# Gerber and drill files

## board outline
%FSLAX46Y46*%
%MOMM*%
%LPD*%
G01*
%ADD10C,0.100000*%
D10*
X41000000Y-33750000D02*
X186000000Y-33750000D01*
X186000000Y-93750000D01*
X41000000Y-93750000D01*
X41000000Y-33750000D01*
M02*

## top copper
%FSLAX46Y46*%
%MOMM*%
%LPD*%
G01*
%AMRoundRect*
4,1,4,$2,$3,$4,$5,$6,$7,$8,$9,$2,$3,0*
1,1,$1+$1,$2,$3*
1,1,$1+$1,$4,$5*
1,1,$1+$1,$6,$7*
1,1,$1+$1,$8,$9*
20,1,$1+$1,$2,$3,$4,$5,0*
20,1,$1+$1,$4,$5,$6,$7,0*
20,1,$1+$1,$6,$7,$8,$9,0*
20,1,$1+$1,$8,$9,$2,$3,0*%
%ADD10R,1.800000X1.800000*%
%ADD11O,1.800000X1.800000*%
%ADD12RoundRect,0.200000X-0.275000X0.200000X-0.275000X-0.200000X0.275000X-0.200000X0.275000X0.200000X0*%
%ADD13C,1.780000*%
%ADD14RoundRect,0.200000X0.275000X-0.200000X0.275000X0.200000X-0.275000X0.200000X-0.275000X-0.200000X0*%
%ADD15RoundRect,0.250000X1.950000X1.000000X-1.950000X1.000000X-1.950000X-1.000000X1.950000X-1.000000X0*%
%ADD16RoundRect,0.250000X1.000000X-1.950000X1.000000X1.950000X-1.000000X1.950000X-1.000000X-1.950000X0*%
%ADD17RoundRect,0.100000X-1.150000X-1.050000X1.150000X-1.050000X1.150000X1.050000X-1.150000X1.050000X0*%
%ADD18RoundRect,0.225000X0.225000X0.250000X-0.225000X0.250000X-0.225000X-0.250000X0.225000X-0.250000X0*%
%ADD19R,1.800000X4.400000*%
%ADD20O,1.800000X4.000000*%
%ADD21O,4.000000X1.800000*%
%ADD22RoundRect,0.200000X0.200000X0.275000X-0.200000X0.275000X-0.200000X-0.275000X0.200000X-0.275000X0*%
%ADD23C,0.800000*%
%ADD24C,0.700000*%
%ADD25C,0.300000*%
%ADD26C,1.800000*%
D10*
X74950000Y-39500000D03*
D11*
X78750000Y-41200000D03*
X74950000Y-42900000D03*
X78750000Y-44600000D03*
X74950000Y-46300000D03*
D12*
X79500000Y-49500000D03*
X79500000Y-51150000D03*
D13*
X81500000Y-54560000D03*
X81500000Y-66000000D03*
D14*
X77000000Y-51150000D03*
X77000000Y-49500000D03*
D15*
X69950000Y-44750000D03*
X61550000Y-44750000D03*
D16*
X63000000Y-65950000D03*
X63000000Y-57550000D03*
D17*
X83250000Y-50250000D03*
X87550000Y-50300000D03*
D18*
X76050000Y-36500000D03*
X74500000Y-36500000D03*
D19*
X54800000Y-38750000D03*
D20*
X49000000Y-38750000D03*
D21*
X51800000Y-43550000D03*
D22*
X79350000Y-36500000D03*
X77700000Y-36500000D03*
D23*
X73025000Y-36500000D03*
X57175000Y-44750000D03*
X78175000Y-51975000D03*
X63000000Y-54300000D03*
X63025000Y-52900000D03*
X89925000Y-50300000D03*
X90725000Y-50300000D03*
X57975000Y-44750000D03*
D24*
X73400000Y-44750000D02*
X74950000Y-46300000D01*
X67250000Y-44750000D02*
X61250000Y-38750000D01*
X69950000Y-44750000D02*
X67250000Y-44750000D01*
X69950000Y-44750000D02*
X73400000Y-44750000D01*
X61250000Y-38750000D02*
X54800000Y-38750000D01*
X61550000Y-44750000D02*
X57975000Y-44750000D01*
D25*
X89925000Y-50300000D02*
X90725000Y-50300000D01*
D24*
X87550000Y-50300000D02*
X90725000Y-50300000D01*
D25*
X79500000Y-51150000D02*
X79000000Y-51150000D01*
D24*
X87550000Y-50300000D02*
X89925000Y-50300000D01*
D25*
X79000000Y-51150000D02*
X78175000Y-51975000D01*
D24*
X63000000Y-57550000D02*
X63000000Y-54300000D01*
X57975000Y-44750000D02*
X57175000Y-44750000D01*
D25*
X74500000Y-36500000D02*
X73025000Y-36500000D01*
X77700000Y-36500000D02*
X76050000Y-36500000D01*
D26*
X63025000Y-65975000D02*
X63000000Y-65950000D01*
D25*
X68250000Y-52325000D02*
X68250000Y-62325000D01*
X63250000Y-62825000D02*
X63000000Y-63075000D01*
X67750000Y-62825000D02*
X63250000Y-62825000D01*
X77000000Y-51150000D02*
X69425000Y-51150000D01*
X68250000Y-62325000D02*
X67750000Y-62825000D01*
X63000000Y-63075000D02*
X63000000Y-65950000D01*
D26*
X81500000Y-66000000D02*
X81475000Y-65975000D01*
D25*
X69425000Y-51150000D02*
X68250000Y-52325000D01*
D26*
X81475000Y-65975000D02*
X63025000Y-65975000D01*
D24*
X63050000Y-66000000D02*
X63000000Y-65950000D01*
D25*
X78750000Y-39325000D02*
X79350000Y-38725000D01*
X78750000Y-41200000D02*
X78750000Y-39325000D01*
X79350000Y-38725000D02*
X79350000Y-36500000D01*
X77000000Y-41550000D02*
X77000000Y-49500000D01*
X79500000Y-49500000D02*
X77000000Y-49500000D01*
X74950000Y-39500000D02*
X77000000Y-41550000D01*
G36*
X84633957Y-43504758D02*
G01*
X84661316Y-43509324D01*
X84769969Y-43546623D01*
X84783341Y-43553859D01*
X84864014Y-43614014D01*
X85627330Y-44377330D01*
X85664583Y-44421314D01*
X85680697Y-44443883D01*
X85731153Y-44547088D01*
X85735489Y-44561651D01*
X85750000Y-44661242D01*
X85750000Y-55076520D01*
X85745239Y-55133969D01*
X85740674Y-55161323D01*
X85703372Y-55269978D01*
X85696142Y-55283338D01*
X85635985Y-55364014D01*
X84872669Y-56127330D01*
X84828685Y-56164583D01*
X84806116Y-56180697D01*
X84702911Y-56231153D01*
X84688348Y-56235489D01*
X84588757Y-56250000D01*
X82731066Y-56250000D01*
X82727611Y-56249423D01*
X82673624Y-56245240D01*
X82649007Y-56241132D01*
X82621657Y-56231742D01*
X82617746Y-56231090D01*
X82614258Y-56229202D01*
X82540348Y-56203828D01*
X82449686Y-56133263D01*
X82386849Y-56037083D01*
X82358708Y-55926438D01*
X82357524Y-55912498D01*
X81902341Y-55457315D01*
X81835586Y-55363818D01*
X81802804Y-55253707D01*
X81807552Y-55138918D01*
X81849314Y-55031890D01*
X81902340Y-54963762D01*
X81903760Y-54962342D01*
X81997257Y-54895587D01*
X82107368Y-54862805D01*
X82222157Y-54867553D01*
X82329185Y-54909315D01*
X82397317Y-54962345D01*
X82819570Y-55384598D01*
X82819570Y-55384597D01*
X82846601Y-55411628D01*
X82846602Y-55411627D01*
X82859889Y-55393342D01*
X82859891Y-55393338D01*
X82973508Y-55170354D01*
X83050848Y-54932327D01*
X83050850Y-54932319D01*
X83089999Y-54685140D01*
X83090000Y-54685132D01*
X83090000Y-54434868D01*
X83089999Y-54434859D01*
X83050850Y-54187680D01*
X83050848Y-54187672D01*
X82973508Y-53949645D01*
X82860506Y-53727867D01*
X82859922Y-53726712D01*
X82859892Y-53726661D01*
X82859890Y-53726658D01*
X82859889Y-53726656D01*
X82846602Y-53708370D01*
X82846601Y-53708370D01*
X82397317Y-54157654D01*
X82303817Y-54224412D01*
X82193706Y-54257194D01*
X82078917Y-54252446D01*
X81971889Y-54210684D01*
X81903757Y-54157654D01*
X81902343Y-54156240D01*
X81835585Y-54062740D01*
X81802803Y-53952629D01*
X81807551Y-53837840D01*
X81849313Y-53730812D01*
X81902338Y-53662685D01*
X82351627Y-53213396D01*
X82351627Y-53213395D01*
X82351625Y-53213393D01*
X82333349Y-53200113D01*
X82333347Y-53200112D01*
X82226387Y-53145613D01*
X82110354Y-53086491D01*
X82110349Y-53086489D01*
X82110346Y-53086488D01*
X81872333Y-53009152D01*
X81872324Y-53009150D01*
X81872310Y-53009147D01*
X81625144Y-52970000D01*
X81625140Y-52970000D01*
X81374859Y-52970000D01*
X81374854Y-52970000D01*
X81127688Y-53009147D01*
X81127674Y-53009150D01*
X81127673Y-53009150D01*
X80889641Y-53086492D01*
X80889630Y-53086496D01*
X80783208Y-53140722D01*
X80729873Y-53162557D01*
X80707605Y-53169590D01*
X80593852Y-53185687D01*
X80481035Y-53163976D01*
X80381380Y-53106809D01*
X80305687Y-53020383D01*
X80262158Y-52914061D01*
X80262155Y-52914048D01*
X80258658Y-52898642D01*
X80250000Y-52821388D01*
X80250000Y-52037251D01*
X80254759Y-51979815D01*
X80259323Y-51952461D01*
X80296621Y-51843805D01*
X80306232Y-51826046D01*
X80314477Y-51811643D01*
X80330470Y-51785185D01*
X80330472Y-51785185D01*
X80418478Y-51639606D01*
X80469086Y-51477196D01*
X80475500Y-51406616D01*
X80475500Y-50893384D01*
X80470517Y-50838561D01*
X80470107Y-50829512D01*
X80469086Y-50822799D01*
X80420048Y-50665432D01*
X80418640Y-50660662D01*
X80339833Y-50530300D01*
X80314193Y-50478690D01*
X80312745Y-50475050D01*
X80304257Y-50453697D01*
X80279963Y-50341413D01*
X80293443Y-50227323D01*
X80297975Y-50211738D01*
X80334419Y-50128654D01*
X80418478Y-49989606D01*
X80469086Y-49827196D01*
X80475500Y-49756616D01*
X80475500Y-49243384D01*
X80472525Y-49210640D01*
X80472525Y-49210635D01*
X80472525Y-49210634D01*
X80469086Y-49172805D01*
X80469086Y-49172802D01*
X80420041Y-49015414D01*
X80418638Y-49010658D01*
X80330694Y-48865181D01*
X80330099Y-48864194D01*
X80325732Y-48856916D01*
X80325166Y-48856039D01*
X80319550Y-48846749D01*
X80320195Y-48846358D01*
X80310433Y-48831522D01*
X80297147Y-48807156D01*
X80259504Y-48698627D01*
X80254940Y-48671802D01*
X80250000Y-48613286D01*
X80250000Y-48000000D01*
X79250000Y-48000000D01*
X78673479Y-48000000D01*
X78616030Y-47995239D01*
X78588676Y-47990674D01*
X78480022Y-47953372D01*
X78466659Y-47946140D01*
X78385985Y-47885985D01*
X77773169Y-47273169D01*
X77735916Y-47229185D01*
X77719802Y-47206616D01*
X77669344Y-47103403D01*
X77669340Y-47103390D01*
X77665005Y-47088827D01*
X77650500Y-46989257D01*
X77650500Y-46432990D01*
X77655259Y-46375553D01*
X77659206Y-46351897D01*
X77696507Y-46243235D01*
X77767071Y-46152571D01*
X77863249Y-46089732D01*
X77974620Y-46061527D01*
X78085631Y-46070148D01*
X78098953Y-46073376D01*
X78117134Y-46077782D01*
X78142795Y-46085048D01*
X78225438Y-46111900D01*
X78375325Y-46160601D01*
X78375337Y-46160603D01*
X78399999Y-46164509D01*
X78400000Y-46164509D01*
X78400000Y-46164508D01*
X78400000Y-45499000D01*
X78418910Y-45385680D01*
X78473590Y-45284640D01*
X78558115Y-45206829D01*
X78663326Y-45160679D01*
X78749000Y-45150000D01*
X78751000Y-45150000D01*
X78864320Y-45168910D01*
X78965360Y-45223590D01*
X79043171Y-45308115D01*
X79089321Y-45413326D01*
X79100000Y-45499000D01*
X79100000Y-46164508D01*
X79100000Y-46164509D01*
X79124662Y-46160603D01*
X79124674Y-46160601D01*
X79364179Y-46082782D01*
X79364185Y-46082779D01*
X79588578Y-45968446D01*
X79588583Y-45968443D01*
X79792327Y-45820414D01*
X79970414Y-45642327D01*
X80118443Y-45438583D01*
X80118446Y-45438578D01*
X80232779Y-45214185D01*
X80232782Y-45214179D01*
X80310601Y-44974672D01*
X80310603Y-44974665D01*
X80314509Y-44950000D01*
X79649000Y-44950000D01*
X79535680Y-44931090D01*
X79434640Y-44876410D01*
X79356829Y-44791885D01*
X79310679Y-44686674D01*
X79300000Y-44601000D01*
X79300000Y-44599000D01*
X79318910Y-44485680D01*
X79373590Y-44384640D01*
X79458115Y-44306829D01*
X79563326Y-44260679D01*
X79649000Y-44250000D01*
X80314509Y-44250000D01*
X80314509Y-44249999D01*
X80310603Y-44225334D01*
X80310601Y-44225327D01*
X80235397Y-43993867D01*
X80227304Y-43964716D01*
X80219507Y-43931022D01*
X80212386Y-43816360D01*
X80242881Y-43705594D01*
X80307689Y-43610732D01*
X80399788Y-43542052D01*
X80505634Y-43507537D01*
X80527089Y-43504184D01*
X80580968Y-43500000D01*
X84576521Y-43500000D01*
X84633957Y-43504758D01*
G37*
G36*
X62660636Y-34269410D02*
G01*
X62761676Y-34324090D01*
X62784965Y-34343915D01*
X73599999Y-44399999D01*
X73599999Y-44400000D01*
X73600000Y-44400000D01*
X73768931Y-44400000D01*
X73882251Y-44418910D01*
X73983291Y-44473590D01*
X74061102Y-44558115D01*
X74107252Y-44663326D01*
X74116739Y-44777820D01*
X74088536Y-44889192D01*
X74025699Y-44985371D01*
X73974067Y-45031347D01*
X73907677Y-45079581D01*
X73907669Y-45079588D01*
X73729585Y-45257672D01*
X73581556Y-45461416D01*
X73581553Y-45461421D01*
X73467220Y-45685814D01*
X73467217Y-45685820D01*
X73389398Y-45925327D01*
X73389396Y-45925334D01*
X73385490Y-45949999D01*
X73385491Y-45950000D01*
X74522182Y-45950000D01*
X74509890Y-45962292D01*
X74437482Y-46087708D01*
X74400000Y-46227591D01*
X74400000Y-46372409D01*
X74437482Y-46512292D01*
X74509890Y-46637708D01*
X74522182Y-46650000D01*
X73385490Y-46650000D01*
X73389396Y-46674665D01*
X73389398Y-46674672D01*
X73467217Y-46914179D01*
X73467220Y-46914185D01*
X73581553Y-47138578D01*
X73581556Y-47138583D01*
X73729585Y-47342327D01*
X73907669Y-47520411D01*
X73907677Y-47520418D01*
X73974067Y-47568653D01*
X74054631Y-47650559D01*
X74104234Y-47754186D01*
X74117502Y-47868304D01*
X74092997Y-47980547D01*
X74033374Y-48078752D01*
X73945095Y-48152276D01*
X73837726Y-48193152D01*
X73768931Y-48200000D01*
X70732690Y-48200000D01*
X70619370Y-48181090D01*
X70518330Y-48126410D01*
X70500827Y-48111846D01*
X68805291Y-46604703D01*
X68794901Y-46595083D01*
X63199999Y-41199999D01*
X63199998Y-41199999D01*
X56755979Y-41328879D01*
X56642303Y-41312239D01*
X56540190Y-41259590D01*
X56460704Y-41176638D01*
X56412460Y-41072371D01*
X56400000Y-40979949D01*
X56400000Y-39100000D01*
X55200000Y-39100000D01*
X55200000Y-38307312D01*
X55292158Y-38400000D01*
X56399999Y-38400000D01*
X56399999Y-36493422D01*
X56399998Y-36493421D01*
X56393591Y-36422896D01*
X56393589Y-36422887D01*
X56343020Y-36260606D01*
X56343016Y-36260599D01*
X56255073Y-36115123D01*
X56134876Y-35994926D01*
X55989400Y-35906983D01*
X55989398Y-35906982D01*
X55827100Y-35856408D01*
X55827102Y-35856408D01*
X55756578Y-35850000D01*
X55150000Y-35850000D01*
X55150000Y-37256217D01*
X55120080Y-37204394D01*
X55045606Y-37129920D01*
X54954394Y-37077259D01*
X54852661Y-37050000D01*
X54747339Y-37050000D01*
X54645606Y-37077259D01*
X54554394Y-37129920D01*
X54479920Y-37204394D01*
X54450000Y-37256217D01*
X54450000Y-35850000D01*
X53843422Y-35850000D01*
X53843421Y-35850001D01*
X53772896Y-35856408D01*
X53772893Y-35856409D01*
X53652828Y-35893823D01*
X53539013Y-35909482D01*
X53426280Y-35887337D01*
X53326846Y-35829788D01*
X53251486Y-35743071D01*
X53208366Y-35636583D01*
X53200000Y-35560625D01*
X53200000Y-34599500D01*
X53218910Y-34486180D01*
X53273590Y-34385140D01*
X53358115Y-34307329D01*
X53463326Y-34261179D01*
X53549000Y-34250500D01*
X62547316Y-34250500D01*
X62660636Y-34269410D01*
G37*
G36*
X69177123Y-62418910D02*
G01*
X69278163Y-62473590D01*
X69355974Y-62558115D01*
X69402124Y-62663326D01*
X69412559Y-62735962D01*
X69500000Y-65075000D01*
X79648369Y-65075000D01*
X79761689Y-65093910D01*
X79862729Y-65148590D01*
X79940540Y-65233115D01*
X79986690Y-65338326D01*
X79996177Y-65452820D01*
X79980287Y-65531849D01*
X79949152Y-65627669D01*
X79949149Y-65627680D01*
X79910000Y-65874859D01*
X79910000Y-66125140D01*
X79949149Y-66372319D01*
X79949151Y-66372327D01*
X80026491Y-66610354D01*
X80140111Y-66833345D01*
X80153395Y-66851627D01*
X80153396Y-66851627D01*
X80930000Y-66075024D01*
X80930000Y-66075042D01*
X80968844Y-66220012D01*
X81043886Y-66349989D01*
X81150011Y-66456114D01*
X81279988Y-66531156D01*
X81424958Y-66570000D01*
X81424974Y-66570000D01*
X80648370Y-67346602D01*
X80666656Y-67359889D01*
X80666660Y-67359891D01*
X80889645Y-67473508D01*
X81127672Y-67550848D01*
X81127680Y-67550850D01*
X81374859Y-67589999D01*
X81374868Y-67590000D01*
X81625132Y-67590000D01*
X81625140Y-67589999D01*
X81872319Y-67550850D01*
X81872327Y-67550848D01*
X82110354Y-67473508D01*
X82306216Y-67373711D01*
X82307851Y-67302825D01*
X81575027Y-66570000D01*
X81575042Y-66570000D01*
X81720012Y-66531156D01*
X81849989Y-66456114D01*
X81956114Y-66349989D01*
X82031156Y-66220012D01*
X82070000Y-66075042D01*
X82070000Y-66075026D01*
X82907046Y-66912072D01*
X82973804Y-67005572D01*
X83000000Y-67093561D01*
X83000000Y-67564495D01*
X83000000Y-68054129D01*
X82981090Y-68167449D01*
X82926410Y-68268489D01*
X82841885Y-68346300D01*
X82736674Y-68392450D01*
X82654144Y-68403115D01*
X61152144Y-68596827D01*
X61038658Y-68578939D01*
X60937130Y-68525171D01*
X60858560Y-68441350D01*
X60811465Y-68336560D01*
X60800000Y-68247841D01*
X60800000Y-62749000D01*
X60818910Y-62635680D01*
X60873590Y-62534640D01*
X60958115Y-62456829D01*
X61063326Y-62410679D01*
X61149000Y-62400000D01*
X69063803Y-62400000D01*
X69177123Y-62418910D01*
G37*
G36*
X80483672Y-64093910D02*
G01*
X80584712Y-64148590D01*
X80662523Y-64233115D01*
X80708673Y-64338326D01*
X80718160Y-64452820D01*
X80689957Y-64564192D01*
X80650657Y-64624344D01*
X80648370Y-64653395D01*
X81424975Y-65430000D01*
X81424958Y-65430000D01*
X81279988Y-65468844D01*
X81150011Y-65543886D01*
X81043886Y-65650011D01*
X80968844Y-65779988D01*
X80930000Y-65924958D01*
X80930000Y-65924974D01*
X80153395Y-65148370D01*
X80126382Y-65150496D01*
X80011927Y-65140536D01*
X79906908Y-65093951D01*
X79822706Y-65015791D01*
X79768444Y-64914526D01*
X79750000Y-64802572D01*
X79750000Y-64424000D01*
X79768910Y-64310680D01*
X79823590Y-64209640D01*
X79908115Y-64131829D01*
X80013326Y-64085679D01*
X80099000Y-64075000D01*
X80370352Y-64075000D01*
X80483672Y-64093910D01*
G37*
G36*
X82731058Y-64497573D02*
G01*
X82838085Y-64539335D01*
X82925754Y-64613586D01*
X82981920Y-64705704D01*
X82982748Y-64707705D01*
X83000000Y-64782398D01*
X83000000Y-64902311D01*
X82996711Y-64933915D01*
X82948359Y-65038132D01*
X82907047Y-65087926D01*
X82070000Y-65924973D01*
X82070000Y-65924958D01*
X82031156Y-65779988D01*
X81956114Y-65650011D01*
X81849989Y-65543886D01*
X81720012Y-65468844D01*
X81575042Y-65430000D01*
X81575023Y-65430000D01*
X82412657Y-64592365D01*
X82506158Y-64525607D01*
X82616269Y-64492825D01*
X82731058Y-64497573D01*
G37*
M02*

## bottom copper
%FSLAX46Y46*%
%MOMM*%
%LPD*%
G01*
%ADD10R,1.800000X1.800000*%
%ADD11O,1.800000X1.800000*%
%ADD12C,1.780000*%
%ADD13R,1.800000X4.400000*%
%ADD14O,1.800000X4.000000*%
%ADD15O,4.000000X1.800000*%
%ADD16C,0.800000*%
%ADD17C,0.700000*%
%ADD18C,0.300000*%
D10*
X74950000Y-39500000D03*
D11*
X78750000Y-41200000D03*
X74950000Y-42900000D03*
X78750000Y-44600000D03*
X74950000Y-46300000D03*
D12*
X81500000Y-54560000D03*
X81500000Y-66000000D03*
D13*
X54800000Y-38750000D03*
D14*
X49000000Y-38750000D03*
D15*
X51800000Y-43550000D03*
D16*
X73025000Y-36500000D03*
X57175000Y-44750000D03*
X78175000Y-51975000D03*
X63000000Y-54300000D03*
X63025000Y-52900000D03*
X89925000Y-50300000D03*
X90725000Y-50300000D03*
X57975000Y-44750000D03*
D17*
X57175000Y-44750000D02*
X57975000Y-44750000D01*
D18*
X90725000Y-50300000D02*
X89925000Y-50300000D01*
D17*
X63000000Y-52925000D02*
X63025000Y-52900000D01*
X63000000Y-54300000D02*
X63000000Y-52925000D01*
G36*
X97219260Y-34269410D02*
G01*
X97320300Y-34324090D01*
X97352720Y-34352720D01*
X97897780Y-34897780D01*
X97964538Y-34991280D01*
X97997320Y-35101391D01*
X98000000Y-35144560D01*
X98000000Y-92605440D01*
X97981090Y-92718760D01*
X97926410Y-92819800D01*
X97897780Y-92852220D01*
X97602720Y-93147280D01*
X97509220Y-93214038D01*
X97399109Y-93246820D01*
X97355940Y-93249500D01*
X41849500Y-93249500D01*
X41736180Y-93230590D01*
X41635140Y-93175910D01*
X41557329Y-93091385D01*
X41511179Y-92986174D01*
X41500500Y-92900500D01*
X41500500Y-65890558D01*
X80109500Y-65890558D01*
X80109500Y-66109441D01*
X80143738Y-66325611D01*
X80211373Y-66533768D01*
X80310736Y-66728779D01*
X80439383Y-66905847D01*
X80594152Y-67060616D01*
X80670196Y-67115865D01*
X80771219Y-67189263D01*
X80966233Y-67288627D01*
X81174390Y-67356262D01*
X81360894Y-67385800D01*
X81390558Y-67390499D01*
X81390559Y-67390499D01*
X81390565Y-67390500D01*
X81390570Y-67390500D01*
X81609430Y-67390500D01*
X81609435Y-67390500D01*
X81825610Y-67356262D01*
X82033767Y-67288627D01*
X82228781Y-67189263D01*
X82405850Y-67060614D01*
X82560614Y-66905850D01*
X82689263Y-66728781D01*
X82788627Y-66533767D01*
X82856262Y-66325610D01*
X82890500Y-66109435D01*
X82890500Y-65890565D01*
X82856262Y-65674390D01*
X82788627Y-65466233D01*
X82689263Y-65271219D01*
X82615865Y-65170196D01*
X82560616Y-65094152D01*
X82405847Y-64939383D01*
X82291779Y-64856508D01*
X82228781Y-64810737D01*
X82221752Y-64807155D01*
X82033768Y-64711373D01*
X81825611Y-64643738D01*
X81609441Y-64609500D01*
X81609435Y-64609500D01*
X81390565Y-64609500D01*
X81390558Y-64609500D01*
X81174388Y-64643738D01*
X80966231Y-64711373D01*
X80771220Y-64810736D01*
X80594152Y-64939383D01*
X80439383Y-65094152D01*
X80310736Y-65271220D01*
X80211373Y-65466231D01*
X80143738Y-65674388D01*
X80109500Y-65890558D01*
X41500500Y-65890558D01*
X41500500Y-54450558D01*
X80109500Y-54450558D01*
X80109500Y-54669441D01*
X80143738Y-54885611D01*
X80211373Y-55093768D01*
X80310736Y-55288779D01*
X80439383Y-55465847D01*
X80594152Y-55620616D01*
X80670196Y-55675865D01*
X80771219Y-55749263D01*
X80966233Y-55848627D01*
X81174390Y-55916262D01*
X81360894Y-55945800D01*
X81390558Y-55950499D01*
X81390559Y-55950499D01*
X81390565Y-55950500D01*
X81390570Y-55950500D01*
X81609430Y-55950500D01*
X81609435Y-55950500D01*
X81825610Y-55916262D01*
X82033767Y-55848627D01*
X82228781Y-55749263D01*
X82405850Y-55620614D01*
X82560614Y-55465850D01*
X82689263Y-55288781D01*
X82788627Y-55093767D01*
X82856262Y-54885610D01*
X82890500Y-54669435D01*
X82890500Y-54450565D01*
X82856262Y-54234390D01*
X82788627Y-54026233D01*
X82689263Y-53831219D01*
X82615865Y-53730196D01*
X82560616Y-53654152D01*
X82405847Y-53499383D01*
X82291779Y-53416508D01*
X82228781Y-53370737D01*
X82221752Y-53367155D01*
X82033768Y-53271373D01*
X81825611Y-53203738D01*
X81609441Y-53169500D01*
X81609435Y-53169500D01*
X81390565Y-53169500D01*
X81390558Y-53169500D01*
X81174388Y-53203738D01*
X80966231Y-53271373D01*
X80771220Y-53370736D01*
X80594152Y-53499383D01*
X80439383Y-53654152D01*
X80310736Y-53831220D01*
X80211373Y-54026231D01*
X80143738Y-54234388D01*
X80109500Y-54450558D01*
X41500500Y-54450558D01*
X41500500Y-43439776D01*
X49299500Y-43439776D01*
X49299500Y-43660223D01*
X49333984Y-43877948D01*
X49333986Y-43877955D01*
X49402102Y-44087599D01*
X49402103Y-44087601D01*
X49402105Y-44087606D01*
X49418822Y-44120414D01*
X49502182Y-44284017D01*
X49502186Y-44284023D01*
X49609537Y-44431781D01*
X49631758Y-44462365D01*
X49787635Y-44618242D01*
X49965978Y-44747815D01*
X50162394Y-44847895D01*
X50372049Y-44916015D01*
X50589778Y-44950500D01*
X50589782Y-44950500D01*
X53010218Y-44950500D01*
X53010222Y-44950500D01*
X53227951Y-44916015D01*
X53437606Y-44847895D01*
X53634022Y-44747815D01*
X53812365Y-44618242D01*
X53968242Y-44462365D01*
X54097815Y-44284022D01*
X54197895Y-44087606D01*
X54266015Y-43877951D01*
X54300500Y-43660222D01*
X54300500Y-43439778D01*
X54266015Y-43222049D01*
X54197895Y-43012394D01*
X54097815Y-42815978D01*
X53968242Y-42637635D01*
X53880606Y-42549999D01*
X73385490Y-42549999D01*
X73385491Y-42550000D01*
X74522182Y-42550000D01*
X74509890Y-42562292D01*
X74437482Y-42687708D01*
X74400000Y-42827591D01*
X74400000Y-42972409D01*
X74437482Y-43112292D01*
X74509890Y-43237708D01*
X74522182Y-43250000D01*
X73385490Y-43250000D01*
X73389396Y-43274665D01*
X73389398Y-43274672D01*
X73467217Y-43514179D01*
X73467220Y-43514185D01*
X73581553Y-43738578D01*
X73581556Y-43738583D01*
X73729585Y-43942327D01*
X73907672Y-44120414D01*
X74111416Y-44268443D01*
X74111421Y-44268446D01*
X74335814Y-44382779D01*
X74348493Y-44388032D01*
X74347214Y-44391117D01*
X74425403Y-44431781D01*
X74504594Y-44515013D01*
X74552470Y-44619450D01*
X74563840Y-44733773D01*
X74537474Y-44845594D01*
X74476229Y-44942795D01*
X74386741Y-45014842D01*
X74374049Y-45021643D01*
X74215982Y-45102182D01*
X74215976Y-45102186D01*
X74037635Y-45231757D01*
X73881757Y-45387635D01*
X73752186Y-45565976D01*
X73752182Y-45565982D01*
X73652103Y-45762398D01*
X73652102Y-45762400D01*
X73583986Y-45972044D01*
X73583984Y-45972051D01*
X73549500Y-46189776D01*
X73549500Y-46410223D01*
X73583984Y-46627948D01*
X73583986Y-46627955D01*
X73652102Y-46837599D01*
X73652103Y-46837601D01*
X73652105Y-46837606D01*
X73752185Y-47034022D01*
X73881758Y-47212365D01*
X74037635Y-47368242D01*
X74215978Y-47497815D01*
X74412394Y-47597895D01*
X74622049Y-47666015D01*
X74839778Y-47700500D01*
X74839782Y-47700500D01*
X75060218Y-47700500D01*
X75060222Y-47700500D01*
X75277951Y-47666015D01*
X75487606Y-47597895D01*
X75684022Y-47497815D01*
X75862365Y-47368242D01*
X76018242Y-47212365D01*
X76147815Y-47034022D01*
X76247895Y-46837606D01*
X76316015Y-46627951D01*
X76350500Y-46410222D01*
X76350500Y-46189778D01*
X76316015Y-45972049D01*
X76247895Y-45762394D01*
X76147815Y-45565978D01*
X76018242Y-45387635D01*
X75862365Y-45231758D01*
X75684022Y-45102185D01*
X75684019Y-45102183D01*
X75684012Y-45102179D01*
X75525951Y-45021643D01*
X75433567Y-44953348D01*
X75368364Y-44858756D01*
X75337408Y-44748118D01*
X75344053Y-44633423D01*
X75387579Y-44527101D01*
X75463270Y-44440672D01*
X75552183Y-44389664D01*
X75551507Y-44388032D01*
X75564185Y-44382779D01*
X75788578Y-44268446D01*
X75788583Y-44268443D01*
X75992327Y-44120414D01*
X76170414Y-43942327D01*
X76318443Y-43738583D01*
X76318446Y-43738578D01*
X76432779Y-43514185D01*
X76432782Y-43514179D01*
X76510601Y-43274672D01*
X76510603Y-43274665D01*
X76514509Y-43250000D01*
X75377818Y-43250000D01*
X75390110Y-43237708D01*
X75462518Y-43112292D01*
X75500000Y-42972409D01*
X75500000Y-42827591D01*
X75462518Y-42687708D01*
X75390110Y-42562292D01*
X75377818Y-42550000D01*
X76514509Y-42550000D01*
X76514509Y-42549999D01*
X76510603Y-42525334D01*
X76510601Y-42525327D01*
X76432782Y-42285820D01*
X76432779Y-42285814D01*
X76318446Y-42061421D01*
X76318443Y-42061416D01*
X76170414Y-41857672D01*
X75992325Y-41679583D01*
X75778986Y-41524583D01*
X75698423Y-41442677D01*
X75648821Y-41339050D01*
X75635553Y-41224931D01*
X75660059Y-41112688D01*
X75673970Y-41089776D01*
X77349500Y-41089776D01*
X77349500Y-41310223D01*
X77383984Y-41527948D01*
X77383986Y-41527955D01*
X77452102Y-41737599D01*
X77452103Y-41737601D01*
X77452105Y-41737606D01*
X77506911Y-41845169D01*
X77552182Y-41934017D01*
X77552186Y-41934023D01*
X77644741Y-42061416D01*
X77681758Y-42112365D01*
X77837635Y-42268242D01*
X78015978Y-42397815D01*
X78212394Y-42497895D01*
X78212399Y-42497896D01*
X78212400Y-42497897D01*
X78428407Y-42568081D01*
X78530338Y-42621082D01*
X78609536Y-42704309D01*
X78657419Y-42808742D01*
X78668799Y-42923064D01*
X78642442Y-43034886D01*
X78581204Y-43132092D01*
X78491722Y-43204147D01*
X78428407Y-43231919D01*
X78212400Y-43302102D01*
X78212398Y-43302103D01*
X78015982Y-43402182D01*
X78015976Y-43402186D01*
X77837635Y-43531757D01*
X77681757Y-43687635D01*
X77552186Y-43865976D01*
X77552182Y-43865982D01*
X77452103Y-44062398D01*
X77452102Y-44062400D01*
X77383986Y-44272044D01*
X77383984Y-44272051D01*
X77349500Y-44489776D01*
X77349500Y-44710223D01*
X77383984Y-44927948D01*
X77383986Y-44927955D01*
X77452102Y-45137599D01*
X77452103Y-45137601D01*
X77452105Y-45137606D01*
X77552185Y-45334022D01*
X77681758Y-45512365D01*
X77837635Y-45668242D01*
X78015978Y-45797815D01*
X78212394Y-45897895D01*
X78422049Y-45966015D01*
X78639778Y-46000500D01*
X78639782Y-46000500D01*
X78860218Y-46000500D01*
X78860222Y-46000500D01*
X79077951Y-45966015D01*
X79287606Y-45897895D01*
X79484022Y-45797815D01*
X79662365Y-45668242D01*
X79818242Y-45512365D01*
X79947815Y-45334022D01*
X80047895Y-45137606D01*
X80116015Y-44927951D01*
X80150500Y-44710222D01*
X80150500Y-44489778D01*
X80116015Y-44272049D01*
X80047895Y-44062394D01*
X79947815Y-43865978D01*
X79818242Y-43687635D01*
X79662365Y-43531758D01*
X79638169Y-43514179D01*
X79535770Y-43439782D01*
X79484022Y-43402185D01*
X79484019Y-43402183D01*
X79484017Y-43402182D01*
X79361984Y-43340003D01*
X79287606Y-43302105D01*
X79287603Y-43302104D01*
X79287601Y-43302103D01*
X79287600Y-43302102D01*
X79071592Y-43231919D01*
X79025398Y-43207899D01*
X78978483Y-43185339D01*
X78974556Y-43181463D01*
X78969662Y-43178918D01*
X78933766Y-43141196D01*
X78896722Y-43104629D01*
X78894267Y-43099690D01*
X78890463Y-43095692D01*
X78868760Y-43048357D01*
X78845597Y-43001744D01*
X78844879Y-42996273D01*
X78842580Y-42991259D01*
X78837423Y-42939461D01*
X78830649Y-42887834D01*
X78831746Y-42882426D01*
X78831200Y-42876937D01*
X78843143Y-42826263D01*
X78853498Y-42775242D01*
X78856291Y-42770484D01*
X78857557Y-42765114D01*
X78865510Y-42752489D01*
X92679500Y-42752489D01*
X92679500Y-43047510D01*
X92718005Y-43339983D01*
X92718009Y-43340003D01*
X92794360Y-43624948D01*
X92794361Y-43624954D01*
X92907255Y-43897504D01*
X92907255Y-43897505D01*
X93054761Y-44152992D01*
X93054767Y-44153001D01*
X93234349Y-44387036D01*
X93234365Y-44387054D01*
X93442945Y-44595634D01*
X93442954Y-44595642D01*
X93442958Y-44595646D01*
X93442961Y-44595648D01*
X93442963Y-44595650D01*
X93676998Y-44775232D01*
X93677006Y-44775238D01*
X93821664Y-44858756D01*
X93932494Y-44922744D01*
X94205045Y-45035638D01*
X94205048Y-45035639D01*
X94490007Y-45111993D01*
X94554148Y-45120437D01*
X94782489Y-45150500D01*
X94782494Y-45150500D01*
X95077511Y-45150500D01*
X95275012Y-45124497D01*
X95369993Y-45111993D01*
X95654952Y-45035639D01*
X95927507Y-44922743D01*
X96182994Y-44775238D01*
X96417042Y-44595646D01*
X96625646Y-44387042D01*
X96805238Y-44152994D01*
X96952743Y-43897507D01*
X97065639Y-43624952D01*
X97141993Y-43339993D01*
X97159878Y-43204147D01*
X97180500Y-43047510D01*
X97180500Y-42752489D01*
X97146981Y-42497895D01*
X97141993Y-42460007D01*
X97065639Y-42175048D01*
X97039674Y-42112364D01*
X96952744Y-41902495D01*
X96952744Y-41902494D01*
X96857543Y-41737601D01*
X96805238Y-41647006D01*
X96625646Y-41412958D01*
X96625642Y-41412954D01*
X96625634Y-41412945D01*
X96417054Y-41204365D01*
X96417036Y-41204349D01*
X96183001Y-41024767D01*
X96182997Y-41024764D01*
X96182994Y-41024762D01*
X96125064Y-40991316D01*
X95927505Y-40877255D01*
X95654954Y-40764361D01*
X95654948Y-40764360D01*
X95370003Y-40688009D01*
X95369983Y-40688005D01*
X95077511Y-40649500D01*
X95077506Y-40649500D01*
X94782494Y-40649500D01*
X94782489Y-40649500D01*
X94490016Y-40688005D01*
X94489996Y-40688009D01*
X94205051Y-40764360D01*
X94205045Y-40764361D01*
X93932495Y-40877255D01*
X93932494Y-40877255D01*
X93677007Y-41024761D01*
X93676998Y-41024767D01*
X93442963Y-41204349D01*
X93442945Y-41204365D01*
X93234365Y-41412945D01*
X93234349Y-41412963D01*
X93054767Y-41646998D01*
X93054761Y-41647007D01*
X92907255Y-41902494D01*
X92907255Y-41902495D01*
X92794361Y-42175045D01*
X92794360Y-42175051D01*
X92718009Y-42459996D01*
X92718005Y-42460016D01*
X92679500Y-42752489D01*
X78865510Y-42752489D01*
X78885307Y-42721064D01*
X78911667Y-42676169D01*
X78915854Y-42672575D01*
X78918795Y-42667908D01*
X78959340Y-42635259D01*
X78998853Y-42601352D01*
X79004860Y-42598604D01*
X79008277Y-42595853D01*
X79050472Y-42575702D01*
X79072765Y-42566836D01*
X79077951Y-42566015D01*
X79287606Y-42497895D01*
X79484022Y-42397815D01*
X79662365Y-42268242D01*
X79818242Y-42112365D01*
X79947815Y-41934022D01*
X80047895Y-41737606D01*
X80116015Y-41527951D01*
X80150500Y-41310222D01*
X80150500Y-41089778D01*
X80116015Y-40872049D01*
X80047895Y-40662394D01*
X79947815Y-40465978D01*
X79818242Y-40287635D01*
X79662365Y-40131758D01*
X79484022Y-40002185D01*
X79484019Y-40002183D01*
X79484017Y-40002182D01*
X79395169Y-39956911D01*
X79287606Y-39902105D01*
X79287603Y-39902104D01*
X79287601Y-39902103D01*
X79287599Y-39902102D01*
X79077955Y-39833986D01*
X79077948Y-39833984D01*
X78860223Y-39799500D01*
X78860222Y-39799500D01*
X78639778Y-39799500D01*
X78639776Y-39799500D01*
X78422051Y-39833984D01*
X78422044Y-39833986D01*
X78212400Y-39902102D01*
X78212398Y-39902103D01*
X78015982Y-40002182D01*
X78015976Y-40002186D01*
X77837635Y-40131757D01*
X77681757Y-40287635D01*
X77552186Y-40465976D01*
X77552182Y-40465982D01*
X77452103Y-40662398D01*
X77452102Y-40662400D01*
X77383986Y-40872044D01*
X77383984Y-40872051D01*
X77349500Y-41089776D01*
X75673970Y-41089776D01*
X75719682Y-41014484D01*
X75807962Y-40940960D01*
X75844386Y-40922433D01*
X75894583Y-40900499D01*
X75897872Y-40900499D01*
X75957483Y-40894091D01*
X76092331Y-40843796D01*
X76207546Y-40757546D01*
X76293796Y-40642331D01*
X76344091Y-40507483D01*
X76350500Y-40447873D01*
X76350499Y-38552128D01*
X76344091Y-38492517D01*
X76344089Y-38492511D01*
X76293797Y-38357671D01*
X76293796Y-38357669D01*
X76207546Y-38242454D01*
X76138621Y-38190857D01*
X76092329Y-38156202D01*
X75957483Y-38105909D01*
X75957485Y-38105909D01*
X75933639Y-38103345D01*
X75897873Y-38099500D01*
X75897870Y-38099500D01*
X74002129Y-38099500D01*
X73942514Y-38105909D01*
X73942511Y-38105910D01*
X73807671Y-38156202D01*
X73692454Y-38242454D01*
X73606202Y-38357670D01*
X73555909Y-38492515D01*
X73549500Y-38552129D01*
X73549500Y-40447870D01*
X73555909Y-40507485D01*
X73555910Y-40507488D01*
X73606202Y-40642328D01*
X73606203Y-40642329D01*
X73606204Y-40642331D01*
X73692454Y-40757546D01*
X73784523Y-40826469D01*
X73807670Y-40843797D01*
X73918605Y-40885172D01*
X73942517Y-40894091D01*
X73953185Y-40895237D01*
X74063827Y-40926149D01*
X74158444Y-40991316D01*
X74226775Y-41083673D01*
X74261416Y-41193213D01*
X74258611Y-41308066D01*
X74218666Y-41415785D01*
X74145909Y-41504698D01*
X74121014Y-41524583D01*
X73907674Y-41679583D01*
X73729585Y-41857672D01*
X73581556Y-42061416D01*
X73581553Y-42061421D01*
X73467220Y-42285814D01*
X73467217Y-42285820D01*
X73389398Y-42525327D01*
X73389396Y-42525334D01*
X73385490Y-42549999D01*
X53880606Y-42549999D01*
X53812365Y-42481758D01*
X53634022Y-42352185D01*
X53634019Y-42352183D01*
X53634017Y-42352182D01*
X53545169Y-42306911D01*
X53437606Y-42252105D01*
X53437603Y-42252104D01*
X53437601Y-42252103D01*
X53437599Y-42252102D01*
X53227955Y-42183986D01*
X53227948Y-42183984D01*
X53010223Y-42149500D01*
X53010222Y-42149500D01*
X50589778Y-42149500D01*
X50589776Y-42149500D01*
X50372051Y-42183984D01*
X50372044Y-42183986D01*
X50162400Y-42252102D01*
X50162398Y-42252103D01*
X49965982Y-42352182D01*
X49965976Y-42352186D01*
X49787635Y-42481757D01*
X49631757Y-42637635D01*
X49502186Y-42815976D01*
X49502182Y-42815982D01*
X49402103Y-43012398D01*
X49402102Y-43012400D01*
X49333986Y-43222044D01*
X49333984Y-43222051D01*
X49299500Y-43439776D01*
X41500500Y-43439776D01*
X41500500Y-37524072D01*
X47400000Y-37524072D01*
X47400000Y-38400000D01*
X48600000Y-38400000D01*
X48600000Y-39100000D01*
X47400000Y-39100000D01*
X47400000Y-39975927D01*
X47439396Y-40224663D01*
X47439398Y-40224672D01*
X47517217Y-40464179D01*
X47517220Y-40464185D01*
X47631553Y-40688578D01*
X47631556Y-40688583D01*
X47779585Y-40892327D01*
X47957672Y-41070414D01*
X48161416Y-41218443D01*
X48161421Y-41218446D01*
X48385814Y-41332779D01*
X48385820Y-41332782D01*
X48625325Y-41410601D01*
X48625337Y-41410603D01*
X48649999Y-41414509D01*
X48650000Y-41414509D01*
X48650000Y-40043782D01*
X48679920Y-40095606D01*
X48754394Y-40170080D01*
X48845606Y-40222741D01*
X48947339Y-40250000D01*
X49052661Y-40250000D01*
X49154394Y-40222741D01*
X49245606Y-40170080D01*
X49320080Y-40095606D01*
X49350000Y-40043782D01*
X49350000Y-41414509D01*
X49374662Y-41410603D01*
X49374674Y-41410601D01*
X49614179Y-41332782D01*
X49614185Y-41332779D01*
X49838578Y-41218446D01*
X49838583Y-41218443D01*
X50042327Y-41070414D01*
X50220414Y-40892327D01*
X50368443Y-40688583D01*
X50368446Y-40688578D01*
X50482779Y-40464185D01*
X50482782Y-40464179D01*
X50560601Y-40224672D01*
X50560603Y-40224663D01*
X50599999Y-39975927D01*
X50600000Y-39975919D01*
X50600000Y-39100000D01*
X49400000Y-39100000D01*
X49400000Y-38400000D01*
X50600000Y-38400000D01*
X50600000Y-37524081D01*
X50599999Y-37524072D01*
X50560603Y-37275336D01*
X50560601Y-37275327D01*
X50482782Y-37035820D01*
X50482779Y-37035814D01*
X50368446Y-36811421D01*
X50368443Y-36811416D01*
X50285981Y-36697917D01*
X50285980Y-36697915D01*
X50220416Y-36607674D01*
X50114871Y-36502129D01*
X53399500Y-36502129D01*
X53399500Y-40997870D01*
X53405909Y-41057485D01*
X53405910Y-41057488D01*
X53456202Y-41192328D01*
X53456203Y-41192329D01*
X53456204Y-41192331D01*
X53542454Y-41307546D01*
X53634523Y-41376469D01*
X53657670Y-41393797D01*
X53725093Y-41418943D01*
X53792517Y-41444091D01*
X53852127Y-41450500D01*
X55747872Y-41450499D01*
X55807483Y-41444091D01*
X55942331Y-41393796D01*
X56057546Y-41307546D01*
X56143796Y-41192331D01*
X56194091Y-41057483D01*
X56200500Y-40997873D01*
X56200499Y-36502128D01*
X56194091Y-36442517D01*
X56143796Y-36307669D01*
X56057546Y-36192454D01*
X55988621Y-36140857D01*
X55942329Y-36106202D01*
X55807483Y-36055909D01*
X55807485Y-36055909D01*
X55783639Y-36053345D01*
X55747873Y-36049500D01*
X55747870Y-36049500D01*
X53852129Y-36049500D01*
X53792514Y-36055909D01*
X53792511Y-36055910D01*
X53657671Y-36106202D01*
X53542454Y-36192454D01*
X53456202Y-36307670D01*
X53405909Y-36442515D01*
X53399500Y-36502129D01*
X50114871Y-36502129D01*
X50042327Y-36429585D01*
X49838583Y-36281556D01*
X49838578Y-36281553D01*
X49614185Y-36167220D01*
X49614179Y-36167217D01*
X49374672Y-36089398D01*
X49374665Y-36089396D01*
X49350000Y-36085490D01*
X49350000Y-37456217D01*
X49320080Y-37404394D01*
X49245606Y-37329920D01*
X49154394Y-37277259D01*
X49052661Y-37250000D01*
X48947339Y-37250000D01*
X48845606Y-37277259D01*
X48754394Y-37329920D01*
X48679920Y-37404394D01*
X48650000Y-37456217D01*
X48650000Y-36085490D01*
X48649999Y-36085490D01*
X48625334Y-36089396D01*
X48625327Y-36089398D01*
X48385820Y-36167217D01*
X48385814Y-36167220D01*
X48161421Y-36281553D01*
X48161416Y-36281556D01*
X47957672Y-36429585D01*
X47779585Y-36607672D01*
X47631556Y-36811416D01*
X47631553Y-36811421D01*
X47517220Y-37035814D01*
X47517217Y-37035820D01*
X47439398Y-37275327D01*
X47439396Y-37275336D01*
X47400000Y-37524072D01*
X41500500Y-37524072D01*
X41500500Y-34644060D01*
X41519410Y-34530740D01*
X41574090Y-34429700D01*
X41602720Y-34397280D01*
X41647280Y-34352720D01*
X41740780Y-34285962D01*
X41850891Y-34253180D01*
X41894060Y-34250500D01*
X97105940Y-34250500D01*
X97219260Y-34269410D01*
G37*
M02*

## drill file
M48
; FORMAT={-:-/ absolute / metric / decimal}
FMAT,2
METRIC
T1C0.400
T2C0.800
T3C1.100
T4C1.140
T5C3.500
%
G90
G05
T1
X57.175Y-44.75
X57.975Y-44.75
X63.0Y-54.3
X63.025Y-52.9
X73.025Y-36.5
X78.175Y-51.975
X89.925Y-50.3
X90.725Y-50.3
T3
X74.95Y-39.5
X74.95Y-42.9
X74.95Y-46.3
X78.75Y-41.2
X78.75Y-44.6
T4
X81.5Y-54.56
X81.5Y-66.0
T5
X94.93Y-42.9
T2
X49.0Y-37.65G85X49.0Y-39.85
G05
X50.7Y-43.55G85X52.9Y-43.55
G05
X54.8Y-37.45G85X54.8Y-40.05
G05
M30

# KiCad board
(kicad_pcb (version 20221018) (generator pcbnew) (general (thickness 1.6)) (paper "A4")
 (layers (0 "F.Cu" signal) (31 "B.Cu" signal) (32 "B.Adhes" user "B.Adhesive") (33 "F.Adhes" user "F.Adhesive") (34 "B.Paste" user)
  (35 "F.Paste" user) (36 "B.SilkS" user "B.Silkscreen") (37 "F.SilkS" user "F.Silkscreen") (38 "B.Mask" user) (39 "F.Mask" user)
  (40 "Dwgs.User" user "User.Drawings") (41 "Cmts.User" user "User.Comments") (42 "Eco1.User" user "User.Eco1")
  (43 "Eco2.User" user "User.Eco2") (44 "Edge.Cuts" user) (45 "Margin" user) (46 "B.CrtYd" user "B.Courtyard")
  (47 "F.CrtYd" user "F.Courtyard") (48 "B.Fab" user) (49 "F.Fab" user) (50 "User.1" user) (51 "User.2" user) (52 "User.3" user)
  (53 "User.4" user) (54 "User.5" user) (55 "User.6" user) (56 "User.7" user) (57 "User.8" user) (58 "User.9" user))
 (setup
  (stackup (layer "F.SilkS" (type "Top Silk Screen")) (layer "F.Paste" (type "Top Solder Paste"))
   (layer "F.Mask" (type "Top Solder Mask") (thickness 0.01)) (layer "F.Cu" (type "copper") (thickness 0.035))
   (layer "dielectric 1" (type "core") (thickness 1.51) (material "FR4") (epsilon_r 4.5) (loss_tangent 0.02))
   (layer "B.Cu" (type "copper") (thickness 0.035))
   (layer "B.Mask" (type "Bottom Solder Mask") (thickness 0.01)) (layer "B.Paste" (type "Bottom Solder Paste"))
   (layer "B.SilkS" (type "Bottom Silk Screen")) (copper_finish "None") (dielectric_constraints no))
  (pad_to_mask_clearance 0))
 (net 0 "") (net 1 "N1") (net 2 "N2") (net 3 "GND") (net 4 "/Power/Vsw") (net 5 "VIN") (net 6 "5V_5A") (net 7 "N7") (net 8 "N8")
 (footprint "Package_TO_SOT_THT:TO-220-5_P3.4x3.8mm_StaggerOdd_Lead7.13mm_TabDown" (layer "F.Cu") (at 74.95 39.5 -90)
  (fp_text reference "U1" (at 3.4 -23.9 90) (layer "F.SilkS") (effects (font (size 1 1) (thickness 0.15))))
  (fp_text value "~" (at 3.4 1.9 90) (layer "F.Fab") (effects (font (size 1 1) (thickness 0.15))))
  (pad "" np_thru_hole oval (at 3.4 -19.98 270) (size 3.5 3.5) (drill 3.5) (layers "*.Cu" "*.Mask"))
  (pad "1" thru_hole rect (at 0 0 270) (size 1.8 1.8) (drill 1.1) (layers "*.Cu" "*.Mask") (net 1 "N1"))
  (pad "2" thru_hole oval (at 1.7 -3.8 270) (size 1.8 1.8) (drill 1.1) (layers "*.Cu" "*.Mask") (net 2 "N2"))
  (pad "3" thru_hole oval (at 3.4 0 270) (size 1.8 1.8) (drill 1.1) (layers "*.Cu" "*.Mask") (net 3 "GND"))
  (pad "4" thru_hole oval (at 5.1 -3.8 270) (size 1.8 1.8) (drill 1.1) (layers "*.Cu" "*.Mask") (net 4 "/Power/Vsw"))
  (pad "5" thru_hole oval (at 6.8 0 270) (size 1.8 1.8) (drill 1.1) (layers "*.Cu" "*.Mask") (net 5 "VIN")))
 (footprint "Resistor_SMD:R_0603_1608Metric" (layer "F.Cu") (at 79.5 50.325 -90)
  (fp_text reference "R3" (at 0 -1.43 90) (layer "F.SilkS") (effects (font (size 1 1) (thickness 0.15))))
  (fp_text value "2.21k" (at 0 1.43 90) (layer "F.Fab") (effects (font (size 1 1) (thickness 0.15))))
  (pad "1" smd roundrect (at -0.825 0 270) (size 0.8 0.95) (layers "F.Cu" "F.Paste" "F.Mask") (roundrect_rratio 0.25) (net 1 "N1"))
  (pad "2" smd roundrect (at 0.825 0 270) (size 0.8 0.95) (layers "F.Cu" "F.Paste" "F.Mask") (roundrect_rratio 0.25) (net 3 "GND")))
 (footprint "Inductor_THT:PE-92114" (layer "F.Cu") (at 81.5 60.28 180)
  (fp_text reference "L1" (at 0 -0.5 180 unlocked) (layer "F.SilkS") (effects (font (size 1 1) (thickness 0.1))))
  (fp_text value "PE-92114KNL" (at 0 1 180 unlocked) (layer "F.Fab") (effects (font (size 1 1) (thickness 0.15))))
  (pad "1" thru_hole circle (at 0 5.72 270) (size 1.78 1.78) (drill 1.14) (layers "*.Cu" "*.Mask") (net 4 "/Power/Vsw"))
  (pad "2" thru_hole circle (at 0 -5.72 270) (size 1.78 1.78) (drill 1.14) (layers "*.Cu" "*.Mask") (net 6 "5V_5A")))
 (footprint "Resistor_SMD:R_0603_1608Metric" (layer "F.Cu") (at 77 50.325 90)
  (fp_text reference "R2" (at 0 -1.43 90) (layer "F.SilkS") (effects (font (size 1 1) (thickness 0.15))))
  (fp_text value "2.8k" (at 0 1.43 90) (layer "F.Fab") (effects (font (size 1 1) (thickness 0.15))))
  (pad "1" smd roundrect (at -0.825 0 90) (size 0.8 0.95) (layers "F.Cu" "F.Paste" "F.Mask") (roundrect_rratio 0.25) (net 6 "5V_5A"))
  (pad "2" smd roundrect (at 0.825 0 90) (size 0.8 0.95) (layers "F.Cu" "F.Paste" "F.Mask") (roundrect_rratio 0.25) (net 1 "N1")))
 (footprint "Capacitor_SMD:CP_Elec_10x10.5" (layer "F.Cu") (at 65.75 44.75 180)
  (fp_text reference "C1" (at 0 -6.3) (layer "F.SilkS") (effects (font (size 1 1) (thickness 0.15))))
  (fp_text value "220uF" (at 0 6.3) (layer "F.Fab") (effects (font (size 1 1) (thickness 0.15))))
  (pad "1" smd roundrect (at -4.2 0 180) (size 4.4 2.5) (layers "F.Cu" "F.Paste" "F.Mask") (roundrect_rratio 0.1) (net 5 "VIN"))
  (pad "2" smd roundrect (at 4.2 0 180) (size 4.4 2.5) (layers "F.Cu" "F.Paste" "F.Mask") (roundrect_rratio 0.1) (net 3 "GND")))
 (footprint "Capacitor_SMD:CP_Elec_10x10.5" (layer "F.Cu") (at 63 61.75 90)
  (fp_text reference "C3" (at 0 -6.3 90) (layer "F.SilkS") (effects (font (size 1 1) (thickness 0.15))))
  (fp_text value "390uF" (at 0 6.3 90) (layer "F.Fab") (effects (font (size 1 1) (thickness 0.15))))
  (pad "1" smd roundrect (at -4.2 0 90) (size 4.4 2.5) (layers "F.Cu" "F.Paste" "F.Mask") (roundrect_rratio 0.1) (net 6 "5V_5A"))
  (pad "2" smd roundrect (at 4.2 0 90) (size 4.4 2.5) (layers "F.Cu" "F.Paste" "F.Mask") (roundrect_rratio 0.1) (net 3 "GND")))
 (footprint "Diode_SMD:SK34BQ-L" (layer "F.Cu") (at 85.4 50.3)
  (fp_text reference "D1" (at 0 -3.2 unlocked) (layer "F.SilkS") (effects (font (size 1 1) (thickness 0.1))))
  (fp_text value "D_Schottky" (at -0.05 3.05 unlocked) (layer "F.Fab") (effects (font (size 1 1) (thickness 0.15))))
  (pad "1" smd roundrect (at -2.15 -0.05) (size 2.5 2.3) (layers "F.Cu" "F.Paste" "F.Mask") (roundrect_rratio 0.04347826087)
   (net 4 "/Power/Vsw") (thermal_bridge_angle 45))
  (pad "2" smd roundrect (at 2.15 0) (size 2.5 2.3) (layers "F.Cu" "F.Paste" "F.Mask") (roundrect_rratio 0.04347826087) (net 3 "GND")
   (thermal_bridge_angle 45)))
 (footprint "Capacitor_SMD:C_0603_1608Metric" (layer "F.Cu") (at 75.275 36.5 180)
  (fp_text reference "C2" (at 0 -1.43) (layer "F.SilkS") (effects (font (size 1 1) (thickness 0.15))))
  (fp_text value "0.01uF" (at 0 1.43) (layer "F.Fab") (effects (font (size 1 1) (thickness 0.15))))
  (pad "1" smd roundrect (at -0.775 0 180) (size 0.9 0.95) (layers "F.Cu" "F.Paste" "F.Mask") (roundrect_rratio 0.25) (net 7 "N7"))
  (pad "2" smd roundrect (at 0.775 0 180) (size 0.9 0.95) (layers "F.Cu" "F.Paste" "F.Mask") (roundrect_rratio 0.25) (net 3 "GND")))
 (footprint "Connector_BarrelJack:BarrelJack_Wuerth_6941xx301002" (layer "F.Cu") (at 54.8 38.75 -90)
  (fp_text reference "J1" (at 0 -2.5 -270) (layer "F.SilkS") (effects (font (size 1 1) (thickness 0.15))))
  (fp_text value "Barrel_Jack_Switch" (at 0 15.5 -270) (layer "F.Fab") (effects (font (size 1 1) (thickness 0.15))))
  (pad "1" thru_hole rect (at 0 0 270) (size 4.4 1.8) (drill oval 3.4 0.8) (layers "*.Cu" "*.Mask") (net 5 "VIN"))
  (pad "2" thru_hole oval (at 0 5.8 270) (size 4 1.8) (drill oval 3 0.8) (layers "*.Cu" "*.Mask") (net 3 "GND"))
  (pad "3" thru_hole oval (at 4.8 3) (size 4 1.8) (drill oval 3 0.8) (layers "*.Cu" "*.Mask") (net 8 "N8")))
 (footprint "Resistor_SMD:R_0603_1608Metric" (layer "F.Cu") (at 78.525 36.5 180)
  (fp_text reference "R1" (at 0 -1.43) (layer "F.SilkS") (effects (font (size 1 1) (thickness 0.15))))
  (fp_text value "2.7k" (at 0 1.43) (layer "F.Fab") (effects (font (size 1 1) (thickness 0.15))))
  (pad "1" smd roundrect (at -0.825 0 180) (size 0.8 0.95) (layers "F.Cu" "F.Paste" "F.Mask") (roundrect_rratio 0.25) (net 2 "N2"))
  (pad "2" smd roundrect (at 0.825 0 180) (size 0.8 0.95) (layers "F.Cu" "F.Paste" "F.Mask") (roundrect_rratio 0.25) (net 7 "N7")))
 (gr_rect (start 41 33.75) (end 186 93.75) (stroke (width 0.1) (type default)) (fill none) (layer "Edge.Cuts"))
 (segment (start 73.4 44.75) (end 74.95 46.3) (width 0.7) (layer "F.Cu") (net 5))
 (segment (start 67.25 44.75) (end 61.25 38.75) (width 0.7) (layer "F.Cu") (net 5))
 (segment (start 69.95 44.75) (end 67.25 44.75) (width 0.7) (layer "F.Cu") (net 5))
 (segment (start 69.95 44.75) (end 73.4 44.75) (width 0.7) (layer "F.Cu") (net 5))
 (segment (start 61.25 38.75) (end 54.8 38.75) (width 0.7) (layer "F.Cu") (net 5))
 (segment (start 61.55 44.75) (end 57.975 44.75) (width 0.7) (layer "F.Cu") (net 3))
 (segment (start 89.925 50.3) (end 90.725 50.3) (width 0.3) (layer "F.Cu") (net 3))
 (segment (start 87.55 50.3) (end 90.725 50.3) (width 0.7) (layer "F.Cu") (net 3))
 (segment (start 79.5 51.15) (end 79 51.15) (width 0.3) (layer "F.Cu") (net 3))
 (segment (start 87.55 50.3) (end 89.925 50.3) (width 0.7) (layer "F.Cu") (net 3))
 (segment (start 79 51.15) (end 78.175 51.975) (width 0.3) (layer "F.Cu") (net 3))
 (segment (start 63 57.55) (end 63 54.3) (width 0.7) (layer "F.Cu") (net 3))
 (segment (start 57.975 44.75) (end 57.175 44.75) (width 0.7) (layer "F.Cu") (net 3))
 (segment (start 74.5 36.5) (end 73.025 36.5) (width 0.3) (layer "F.Cu") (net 3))
 (via (at 73.025 36.5) (size 0.8) (drill 0.4) (layers "F.Cu" "B.Cu") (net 3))
 (via (at 57.175 44.75) (size 0.8) (drill 0.4) (layers "F.Cu" "B.Cu") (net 3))
 (via (at 78.175 51.975) (size 0.8) (drill 0.4) (layers "F.Cu" "B.Cu") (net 3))
 (via (at 63 54.3) (size 0.8) (drill 0.4) (layers "F.Cu" "B.Cu") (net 3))
 (via (at 63.025 52.9) (size 0.8) (drill 0.4) (layers "F.Cu" "B.Cu") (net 3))
 (via (at 89.925 50.3) (size 0.8) (drill 0.4) (layers "F.Cu" "B.Cu") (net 3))
 (via (at 90.725 50.3) (size 0.8) (drill 0.4) (layers "F.Cu" "B.Cu") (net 3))
 (via (at 57.975 44.75) (size 0.8) (drill 0.4) (layers "F.Cu" "B.Cu") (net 3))
 (segment (start 57.175 44.75) (end 57.975 44.75) (width 0.7) (layer "B.Cu") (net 3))
 (segment (start 90.725 50.3) (end 89.925 50.3) (width 0.3) (layer "B.Cu") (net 3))
 (segment (start 63 52.925) (end 63.025 52.9) (width 0.7) (layer "B.Cu") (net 3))
 (segment (start 63 54.3) (end 63 52.925) (width 0.7) (layer "B.Cu") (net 3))
 (segment (start 77.7 36.5) (end 76.05 36.5) (width 0.3) (layer "F.Cu") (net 7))
 (segment (start 63.025 65.975) (end 63 65.95) (width 1.8) (layer "F.Cu") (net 6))
 (segment (start 68.25 52.325) (end 68.25 62.325) (width 0.3) (layer "F.Cu") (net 6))
 (segment (start 63.25 62.825) (end 63 63.075) (width 0.3) (layer "F.Cu") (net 6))
 (segment (start 67.75 62.825) (end 63.25 62.825) (width 0.3) (layer "F.Cu") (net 6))
 (segment (start 77 51.15) (end 69.425 51.15) (width 0.3) (layer "F.Cu") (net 6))
 (segment (start 68.25 62.325) (end 67.75 62.825) (width 0.3) (layer "F.Cu") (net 6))
 (segment (start 63 63.075) (end 63 65.95) (width 0.3) (layer "F.Cu") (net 6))
 (segment (start 81.5 66) (end 81.475 65.975) (width 1.8) (layer "F.Cu") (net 6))
 (segment (start 69.425 51.15) (end 68.25 52.325) (width 0.3) (layer "F.Cu") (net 6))
 (segment (start 81.475 65.975) (end 63.025 65.975) (width 1.8) (layer "F.Cu") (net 6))
 (segment (start 63.05 66) (end 63 65.95) (width 0.7) (layer "F.Cu") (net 6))
 (segment (start 78.75 39.325) (end 79.35 38.725) (width 0.3) (layer "F.Cu") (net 2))
 (segment (start 78.75 41.2) (end 78.75 39.325) (width 0.3) (layer "F.Cu") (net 2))
 (segment (start 79.35 38.725) (end 79.35 36.5) (width 0.3) (layer "F.Cu") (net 2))
 (segment (start 77 41.55) (end 77 49.5) (width 0.3) (layer "F.Cu") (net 1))
 (segment (start 79.5 49.5) (end 77 49.5) (width 0.3) (layer "F.Cu") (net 1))
 (segment (start 74.95 39.5) (end 77 41.55) (width 0.3) (layer "F.Cu") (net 1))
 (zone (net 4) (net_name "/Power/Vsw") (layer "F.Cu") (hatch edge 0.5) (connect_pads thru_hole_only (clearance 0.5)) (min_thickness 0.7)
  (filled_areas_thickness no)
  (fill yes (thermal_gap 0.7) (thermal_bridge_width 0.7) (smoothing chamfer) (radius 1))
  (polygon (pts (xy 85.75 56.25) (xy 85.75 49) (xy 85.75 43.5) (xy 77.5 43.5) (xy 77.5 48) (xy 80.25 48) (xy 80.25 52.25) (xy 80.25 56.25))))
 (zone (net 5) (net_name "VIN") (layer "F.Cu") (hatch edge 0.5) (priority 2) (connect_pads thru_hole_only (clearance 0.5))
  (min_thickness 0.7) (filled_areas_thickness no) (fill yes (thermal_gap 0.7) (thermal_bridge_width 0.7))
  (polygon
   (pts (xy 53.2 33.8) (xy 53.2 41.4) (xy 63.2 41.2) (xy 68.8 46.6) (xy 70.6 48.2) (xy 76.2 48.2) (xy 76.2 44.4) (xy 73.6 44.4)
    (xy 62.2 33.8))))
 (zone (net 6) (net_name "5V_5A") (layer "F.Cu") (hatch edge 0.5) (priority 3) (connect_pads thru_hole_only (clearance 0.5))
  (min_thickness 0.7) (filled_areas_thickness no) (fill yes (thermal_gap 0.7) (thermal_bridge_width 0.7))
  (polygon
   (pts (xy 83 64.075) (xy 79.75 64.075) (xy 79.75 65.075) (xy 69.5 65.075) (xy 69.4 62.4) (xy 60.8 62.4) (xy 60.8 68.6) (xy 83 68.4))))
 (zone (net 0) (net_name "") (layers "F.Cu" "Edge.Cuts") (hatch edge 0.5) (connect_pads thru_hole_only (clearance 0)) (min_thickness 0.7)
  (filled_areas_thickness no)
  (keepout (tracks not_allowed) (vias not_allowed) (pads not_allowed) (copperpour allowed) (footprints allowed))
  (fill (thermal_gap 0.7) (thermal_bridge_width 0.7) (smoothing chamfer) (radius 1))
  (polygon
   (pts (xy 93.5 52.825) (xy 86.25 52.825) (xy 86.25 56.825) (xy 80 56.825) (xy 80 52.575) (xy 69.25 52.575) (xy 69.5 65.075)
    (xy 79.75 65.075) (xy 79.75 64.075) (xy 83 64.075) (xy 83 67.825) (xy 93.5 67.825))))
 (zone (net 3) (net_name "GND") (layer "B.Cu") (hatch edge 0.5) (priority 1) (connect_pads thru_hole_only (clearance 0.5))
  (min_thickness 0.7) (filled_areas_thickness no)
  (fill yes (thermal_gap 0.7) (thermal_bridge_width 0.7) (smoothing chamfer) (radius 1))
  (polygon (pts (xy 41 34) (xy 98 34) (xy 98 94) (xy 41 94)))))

